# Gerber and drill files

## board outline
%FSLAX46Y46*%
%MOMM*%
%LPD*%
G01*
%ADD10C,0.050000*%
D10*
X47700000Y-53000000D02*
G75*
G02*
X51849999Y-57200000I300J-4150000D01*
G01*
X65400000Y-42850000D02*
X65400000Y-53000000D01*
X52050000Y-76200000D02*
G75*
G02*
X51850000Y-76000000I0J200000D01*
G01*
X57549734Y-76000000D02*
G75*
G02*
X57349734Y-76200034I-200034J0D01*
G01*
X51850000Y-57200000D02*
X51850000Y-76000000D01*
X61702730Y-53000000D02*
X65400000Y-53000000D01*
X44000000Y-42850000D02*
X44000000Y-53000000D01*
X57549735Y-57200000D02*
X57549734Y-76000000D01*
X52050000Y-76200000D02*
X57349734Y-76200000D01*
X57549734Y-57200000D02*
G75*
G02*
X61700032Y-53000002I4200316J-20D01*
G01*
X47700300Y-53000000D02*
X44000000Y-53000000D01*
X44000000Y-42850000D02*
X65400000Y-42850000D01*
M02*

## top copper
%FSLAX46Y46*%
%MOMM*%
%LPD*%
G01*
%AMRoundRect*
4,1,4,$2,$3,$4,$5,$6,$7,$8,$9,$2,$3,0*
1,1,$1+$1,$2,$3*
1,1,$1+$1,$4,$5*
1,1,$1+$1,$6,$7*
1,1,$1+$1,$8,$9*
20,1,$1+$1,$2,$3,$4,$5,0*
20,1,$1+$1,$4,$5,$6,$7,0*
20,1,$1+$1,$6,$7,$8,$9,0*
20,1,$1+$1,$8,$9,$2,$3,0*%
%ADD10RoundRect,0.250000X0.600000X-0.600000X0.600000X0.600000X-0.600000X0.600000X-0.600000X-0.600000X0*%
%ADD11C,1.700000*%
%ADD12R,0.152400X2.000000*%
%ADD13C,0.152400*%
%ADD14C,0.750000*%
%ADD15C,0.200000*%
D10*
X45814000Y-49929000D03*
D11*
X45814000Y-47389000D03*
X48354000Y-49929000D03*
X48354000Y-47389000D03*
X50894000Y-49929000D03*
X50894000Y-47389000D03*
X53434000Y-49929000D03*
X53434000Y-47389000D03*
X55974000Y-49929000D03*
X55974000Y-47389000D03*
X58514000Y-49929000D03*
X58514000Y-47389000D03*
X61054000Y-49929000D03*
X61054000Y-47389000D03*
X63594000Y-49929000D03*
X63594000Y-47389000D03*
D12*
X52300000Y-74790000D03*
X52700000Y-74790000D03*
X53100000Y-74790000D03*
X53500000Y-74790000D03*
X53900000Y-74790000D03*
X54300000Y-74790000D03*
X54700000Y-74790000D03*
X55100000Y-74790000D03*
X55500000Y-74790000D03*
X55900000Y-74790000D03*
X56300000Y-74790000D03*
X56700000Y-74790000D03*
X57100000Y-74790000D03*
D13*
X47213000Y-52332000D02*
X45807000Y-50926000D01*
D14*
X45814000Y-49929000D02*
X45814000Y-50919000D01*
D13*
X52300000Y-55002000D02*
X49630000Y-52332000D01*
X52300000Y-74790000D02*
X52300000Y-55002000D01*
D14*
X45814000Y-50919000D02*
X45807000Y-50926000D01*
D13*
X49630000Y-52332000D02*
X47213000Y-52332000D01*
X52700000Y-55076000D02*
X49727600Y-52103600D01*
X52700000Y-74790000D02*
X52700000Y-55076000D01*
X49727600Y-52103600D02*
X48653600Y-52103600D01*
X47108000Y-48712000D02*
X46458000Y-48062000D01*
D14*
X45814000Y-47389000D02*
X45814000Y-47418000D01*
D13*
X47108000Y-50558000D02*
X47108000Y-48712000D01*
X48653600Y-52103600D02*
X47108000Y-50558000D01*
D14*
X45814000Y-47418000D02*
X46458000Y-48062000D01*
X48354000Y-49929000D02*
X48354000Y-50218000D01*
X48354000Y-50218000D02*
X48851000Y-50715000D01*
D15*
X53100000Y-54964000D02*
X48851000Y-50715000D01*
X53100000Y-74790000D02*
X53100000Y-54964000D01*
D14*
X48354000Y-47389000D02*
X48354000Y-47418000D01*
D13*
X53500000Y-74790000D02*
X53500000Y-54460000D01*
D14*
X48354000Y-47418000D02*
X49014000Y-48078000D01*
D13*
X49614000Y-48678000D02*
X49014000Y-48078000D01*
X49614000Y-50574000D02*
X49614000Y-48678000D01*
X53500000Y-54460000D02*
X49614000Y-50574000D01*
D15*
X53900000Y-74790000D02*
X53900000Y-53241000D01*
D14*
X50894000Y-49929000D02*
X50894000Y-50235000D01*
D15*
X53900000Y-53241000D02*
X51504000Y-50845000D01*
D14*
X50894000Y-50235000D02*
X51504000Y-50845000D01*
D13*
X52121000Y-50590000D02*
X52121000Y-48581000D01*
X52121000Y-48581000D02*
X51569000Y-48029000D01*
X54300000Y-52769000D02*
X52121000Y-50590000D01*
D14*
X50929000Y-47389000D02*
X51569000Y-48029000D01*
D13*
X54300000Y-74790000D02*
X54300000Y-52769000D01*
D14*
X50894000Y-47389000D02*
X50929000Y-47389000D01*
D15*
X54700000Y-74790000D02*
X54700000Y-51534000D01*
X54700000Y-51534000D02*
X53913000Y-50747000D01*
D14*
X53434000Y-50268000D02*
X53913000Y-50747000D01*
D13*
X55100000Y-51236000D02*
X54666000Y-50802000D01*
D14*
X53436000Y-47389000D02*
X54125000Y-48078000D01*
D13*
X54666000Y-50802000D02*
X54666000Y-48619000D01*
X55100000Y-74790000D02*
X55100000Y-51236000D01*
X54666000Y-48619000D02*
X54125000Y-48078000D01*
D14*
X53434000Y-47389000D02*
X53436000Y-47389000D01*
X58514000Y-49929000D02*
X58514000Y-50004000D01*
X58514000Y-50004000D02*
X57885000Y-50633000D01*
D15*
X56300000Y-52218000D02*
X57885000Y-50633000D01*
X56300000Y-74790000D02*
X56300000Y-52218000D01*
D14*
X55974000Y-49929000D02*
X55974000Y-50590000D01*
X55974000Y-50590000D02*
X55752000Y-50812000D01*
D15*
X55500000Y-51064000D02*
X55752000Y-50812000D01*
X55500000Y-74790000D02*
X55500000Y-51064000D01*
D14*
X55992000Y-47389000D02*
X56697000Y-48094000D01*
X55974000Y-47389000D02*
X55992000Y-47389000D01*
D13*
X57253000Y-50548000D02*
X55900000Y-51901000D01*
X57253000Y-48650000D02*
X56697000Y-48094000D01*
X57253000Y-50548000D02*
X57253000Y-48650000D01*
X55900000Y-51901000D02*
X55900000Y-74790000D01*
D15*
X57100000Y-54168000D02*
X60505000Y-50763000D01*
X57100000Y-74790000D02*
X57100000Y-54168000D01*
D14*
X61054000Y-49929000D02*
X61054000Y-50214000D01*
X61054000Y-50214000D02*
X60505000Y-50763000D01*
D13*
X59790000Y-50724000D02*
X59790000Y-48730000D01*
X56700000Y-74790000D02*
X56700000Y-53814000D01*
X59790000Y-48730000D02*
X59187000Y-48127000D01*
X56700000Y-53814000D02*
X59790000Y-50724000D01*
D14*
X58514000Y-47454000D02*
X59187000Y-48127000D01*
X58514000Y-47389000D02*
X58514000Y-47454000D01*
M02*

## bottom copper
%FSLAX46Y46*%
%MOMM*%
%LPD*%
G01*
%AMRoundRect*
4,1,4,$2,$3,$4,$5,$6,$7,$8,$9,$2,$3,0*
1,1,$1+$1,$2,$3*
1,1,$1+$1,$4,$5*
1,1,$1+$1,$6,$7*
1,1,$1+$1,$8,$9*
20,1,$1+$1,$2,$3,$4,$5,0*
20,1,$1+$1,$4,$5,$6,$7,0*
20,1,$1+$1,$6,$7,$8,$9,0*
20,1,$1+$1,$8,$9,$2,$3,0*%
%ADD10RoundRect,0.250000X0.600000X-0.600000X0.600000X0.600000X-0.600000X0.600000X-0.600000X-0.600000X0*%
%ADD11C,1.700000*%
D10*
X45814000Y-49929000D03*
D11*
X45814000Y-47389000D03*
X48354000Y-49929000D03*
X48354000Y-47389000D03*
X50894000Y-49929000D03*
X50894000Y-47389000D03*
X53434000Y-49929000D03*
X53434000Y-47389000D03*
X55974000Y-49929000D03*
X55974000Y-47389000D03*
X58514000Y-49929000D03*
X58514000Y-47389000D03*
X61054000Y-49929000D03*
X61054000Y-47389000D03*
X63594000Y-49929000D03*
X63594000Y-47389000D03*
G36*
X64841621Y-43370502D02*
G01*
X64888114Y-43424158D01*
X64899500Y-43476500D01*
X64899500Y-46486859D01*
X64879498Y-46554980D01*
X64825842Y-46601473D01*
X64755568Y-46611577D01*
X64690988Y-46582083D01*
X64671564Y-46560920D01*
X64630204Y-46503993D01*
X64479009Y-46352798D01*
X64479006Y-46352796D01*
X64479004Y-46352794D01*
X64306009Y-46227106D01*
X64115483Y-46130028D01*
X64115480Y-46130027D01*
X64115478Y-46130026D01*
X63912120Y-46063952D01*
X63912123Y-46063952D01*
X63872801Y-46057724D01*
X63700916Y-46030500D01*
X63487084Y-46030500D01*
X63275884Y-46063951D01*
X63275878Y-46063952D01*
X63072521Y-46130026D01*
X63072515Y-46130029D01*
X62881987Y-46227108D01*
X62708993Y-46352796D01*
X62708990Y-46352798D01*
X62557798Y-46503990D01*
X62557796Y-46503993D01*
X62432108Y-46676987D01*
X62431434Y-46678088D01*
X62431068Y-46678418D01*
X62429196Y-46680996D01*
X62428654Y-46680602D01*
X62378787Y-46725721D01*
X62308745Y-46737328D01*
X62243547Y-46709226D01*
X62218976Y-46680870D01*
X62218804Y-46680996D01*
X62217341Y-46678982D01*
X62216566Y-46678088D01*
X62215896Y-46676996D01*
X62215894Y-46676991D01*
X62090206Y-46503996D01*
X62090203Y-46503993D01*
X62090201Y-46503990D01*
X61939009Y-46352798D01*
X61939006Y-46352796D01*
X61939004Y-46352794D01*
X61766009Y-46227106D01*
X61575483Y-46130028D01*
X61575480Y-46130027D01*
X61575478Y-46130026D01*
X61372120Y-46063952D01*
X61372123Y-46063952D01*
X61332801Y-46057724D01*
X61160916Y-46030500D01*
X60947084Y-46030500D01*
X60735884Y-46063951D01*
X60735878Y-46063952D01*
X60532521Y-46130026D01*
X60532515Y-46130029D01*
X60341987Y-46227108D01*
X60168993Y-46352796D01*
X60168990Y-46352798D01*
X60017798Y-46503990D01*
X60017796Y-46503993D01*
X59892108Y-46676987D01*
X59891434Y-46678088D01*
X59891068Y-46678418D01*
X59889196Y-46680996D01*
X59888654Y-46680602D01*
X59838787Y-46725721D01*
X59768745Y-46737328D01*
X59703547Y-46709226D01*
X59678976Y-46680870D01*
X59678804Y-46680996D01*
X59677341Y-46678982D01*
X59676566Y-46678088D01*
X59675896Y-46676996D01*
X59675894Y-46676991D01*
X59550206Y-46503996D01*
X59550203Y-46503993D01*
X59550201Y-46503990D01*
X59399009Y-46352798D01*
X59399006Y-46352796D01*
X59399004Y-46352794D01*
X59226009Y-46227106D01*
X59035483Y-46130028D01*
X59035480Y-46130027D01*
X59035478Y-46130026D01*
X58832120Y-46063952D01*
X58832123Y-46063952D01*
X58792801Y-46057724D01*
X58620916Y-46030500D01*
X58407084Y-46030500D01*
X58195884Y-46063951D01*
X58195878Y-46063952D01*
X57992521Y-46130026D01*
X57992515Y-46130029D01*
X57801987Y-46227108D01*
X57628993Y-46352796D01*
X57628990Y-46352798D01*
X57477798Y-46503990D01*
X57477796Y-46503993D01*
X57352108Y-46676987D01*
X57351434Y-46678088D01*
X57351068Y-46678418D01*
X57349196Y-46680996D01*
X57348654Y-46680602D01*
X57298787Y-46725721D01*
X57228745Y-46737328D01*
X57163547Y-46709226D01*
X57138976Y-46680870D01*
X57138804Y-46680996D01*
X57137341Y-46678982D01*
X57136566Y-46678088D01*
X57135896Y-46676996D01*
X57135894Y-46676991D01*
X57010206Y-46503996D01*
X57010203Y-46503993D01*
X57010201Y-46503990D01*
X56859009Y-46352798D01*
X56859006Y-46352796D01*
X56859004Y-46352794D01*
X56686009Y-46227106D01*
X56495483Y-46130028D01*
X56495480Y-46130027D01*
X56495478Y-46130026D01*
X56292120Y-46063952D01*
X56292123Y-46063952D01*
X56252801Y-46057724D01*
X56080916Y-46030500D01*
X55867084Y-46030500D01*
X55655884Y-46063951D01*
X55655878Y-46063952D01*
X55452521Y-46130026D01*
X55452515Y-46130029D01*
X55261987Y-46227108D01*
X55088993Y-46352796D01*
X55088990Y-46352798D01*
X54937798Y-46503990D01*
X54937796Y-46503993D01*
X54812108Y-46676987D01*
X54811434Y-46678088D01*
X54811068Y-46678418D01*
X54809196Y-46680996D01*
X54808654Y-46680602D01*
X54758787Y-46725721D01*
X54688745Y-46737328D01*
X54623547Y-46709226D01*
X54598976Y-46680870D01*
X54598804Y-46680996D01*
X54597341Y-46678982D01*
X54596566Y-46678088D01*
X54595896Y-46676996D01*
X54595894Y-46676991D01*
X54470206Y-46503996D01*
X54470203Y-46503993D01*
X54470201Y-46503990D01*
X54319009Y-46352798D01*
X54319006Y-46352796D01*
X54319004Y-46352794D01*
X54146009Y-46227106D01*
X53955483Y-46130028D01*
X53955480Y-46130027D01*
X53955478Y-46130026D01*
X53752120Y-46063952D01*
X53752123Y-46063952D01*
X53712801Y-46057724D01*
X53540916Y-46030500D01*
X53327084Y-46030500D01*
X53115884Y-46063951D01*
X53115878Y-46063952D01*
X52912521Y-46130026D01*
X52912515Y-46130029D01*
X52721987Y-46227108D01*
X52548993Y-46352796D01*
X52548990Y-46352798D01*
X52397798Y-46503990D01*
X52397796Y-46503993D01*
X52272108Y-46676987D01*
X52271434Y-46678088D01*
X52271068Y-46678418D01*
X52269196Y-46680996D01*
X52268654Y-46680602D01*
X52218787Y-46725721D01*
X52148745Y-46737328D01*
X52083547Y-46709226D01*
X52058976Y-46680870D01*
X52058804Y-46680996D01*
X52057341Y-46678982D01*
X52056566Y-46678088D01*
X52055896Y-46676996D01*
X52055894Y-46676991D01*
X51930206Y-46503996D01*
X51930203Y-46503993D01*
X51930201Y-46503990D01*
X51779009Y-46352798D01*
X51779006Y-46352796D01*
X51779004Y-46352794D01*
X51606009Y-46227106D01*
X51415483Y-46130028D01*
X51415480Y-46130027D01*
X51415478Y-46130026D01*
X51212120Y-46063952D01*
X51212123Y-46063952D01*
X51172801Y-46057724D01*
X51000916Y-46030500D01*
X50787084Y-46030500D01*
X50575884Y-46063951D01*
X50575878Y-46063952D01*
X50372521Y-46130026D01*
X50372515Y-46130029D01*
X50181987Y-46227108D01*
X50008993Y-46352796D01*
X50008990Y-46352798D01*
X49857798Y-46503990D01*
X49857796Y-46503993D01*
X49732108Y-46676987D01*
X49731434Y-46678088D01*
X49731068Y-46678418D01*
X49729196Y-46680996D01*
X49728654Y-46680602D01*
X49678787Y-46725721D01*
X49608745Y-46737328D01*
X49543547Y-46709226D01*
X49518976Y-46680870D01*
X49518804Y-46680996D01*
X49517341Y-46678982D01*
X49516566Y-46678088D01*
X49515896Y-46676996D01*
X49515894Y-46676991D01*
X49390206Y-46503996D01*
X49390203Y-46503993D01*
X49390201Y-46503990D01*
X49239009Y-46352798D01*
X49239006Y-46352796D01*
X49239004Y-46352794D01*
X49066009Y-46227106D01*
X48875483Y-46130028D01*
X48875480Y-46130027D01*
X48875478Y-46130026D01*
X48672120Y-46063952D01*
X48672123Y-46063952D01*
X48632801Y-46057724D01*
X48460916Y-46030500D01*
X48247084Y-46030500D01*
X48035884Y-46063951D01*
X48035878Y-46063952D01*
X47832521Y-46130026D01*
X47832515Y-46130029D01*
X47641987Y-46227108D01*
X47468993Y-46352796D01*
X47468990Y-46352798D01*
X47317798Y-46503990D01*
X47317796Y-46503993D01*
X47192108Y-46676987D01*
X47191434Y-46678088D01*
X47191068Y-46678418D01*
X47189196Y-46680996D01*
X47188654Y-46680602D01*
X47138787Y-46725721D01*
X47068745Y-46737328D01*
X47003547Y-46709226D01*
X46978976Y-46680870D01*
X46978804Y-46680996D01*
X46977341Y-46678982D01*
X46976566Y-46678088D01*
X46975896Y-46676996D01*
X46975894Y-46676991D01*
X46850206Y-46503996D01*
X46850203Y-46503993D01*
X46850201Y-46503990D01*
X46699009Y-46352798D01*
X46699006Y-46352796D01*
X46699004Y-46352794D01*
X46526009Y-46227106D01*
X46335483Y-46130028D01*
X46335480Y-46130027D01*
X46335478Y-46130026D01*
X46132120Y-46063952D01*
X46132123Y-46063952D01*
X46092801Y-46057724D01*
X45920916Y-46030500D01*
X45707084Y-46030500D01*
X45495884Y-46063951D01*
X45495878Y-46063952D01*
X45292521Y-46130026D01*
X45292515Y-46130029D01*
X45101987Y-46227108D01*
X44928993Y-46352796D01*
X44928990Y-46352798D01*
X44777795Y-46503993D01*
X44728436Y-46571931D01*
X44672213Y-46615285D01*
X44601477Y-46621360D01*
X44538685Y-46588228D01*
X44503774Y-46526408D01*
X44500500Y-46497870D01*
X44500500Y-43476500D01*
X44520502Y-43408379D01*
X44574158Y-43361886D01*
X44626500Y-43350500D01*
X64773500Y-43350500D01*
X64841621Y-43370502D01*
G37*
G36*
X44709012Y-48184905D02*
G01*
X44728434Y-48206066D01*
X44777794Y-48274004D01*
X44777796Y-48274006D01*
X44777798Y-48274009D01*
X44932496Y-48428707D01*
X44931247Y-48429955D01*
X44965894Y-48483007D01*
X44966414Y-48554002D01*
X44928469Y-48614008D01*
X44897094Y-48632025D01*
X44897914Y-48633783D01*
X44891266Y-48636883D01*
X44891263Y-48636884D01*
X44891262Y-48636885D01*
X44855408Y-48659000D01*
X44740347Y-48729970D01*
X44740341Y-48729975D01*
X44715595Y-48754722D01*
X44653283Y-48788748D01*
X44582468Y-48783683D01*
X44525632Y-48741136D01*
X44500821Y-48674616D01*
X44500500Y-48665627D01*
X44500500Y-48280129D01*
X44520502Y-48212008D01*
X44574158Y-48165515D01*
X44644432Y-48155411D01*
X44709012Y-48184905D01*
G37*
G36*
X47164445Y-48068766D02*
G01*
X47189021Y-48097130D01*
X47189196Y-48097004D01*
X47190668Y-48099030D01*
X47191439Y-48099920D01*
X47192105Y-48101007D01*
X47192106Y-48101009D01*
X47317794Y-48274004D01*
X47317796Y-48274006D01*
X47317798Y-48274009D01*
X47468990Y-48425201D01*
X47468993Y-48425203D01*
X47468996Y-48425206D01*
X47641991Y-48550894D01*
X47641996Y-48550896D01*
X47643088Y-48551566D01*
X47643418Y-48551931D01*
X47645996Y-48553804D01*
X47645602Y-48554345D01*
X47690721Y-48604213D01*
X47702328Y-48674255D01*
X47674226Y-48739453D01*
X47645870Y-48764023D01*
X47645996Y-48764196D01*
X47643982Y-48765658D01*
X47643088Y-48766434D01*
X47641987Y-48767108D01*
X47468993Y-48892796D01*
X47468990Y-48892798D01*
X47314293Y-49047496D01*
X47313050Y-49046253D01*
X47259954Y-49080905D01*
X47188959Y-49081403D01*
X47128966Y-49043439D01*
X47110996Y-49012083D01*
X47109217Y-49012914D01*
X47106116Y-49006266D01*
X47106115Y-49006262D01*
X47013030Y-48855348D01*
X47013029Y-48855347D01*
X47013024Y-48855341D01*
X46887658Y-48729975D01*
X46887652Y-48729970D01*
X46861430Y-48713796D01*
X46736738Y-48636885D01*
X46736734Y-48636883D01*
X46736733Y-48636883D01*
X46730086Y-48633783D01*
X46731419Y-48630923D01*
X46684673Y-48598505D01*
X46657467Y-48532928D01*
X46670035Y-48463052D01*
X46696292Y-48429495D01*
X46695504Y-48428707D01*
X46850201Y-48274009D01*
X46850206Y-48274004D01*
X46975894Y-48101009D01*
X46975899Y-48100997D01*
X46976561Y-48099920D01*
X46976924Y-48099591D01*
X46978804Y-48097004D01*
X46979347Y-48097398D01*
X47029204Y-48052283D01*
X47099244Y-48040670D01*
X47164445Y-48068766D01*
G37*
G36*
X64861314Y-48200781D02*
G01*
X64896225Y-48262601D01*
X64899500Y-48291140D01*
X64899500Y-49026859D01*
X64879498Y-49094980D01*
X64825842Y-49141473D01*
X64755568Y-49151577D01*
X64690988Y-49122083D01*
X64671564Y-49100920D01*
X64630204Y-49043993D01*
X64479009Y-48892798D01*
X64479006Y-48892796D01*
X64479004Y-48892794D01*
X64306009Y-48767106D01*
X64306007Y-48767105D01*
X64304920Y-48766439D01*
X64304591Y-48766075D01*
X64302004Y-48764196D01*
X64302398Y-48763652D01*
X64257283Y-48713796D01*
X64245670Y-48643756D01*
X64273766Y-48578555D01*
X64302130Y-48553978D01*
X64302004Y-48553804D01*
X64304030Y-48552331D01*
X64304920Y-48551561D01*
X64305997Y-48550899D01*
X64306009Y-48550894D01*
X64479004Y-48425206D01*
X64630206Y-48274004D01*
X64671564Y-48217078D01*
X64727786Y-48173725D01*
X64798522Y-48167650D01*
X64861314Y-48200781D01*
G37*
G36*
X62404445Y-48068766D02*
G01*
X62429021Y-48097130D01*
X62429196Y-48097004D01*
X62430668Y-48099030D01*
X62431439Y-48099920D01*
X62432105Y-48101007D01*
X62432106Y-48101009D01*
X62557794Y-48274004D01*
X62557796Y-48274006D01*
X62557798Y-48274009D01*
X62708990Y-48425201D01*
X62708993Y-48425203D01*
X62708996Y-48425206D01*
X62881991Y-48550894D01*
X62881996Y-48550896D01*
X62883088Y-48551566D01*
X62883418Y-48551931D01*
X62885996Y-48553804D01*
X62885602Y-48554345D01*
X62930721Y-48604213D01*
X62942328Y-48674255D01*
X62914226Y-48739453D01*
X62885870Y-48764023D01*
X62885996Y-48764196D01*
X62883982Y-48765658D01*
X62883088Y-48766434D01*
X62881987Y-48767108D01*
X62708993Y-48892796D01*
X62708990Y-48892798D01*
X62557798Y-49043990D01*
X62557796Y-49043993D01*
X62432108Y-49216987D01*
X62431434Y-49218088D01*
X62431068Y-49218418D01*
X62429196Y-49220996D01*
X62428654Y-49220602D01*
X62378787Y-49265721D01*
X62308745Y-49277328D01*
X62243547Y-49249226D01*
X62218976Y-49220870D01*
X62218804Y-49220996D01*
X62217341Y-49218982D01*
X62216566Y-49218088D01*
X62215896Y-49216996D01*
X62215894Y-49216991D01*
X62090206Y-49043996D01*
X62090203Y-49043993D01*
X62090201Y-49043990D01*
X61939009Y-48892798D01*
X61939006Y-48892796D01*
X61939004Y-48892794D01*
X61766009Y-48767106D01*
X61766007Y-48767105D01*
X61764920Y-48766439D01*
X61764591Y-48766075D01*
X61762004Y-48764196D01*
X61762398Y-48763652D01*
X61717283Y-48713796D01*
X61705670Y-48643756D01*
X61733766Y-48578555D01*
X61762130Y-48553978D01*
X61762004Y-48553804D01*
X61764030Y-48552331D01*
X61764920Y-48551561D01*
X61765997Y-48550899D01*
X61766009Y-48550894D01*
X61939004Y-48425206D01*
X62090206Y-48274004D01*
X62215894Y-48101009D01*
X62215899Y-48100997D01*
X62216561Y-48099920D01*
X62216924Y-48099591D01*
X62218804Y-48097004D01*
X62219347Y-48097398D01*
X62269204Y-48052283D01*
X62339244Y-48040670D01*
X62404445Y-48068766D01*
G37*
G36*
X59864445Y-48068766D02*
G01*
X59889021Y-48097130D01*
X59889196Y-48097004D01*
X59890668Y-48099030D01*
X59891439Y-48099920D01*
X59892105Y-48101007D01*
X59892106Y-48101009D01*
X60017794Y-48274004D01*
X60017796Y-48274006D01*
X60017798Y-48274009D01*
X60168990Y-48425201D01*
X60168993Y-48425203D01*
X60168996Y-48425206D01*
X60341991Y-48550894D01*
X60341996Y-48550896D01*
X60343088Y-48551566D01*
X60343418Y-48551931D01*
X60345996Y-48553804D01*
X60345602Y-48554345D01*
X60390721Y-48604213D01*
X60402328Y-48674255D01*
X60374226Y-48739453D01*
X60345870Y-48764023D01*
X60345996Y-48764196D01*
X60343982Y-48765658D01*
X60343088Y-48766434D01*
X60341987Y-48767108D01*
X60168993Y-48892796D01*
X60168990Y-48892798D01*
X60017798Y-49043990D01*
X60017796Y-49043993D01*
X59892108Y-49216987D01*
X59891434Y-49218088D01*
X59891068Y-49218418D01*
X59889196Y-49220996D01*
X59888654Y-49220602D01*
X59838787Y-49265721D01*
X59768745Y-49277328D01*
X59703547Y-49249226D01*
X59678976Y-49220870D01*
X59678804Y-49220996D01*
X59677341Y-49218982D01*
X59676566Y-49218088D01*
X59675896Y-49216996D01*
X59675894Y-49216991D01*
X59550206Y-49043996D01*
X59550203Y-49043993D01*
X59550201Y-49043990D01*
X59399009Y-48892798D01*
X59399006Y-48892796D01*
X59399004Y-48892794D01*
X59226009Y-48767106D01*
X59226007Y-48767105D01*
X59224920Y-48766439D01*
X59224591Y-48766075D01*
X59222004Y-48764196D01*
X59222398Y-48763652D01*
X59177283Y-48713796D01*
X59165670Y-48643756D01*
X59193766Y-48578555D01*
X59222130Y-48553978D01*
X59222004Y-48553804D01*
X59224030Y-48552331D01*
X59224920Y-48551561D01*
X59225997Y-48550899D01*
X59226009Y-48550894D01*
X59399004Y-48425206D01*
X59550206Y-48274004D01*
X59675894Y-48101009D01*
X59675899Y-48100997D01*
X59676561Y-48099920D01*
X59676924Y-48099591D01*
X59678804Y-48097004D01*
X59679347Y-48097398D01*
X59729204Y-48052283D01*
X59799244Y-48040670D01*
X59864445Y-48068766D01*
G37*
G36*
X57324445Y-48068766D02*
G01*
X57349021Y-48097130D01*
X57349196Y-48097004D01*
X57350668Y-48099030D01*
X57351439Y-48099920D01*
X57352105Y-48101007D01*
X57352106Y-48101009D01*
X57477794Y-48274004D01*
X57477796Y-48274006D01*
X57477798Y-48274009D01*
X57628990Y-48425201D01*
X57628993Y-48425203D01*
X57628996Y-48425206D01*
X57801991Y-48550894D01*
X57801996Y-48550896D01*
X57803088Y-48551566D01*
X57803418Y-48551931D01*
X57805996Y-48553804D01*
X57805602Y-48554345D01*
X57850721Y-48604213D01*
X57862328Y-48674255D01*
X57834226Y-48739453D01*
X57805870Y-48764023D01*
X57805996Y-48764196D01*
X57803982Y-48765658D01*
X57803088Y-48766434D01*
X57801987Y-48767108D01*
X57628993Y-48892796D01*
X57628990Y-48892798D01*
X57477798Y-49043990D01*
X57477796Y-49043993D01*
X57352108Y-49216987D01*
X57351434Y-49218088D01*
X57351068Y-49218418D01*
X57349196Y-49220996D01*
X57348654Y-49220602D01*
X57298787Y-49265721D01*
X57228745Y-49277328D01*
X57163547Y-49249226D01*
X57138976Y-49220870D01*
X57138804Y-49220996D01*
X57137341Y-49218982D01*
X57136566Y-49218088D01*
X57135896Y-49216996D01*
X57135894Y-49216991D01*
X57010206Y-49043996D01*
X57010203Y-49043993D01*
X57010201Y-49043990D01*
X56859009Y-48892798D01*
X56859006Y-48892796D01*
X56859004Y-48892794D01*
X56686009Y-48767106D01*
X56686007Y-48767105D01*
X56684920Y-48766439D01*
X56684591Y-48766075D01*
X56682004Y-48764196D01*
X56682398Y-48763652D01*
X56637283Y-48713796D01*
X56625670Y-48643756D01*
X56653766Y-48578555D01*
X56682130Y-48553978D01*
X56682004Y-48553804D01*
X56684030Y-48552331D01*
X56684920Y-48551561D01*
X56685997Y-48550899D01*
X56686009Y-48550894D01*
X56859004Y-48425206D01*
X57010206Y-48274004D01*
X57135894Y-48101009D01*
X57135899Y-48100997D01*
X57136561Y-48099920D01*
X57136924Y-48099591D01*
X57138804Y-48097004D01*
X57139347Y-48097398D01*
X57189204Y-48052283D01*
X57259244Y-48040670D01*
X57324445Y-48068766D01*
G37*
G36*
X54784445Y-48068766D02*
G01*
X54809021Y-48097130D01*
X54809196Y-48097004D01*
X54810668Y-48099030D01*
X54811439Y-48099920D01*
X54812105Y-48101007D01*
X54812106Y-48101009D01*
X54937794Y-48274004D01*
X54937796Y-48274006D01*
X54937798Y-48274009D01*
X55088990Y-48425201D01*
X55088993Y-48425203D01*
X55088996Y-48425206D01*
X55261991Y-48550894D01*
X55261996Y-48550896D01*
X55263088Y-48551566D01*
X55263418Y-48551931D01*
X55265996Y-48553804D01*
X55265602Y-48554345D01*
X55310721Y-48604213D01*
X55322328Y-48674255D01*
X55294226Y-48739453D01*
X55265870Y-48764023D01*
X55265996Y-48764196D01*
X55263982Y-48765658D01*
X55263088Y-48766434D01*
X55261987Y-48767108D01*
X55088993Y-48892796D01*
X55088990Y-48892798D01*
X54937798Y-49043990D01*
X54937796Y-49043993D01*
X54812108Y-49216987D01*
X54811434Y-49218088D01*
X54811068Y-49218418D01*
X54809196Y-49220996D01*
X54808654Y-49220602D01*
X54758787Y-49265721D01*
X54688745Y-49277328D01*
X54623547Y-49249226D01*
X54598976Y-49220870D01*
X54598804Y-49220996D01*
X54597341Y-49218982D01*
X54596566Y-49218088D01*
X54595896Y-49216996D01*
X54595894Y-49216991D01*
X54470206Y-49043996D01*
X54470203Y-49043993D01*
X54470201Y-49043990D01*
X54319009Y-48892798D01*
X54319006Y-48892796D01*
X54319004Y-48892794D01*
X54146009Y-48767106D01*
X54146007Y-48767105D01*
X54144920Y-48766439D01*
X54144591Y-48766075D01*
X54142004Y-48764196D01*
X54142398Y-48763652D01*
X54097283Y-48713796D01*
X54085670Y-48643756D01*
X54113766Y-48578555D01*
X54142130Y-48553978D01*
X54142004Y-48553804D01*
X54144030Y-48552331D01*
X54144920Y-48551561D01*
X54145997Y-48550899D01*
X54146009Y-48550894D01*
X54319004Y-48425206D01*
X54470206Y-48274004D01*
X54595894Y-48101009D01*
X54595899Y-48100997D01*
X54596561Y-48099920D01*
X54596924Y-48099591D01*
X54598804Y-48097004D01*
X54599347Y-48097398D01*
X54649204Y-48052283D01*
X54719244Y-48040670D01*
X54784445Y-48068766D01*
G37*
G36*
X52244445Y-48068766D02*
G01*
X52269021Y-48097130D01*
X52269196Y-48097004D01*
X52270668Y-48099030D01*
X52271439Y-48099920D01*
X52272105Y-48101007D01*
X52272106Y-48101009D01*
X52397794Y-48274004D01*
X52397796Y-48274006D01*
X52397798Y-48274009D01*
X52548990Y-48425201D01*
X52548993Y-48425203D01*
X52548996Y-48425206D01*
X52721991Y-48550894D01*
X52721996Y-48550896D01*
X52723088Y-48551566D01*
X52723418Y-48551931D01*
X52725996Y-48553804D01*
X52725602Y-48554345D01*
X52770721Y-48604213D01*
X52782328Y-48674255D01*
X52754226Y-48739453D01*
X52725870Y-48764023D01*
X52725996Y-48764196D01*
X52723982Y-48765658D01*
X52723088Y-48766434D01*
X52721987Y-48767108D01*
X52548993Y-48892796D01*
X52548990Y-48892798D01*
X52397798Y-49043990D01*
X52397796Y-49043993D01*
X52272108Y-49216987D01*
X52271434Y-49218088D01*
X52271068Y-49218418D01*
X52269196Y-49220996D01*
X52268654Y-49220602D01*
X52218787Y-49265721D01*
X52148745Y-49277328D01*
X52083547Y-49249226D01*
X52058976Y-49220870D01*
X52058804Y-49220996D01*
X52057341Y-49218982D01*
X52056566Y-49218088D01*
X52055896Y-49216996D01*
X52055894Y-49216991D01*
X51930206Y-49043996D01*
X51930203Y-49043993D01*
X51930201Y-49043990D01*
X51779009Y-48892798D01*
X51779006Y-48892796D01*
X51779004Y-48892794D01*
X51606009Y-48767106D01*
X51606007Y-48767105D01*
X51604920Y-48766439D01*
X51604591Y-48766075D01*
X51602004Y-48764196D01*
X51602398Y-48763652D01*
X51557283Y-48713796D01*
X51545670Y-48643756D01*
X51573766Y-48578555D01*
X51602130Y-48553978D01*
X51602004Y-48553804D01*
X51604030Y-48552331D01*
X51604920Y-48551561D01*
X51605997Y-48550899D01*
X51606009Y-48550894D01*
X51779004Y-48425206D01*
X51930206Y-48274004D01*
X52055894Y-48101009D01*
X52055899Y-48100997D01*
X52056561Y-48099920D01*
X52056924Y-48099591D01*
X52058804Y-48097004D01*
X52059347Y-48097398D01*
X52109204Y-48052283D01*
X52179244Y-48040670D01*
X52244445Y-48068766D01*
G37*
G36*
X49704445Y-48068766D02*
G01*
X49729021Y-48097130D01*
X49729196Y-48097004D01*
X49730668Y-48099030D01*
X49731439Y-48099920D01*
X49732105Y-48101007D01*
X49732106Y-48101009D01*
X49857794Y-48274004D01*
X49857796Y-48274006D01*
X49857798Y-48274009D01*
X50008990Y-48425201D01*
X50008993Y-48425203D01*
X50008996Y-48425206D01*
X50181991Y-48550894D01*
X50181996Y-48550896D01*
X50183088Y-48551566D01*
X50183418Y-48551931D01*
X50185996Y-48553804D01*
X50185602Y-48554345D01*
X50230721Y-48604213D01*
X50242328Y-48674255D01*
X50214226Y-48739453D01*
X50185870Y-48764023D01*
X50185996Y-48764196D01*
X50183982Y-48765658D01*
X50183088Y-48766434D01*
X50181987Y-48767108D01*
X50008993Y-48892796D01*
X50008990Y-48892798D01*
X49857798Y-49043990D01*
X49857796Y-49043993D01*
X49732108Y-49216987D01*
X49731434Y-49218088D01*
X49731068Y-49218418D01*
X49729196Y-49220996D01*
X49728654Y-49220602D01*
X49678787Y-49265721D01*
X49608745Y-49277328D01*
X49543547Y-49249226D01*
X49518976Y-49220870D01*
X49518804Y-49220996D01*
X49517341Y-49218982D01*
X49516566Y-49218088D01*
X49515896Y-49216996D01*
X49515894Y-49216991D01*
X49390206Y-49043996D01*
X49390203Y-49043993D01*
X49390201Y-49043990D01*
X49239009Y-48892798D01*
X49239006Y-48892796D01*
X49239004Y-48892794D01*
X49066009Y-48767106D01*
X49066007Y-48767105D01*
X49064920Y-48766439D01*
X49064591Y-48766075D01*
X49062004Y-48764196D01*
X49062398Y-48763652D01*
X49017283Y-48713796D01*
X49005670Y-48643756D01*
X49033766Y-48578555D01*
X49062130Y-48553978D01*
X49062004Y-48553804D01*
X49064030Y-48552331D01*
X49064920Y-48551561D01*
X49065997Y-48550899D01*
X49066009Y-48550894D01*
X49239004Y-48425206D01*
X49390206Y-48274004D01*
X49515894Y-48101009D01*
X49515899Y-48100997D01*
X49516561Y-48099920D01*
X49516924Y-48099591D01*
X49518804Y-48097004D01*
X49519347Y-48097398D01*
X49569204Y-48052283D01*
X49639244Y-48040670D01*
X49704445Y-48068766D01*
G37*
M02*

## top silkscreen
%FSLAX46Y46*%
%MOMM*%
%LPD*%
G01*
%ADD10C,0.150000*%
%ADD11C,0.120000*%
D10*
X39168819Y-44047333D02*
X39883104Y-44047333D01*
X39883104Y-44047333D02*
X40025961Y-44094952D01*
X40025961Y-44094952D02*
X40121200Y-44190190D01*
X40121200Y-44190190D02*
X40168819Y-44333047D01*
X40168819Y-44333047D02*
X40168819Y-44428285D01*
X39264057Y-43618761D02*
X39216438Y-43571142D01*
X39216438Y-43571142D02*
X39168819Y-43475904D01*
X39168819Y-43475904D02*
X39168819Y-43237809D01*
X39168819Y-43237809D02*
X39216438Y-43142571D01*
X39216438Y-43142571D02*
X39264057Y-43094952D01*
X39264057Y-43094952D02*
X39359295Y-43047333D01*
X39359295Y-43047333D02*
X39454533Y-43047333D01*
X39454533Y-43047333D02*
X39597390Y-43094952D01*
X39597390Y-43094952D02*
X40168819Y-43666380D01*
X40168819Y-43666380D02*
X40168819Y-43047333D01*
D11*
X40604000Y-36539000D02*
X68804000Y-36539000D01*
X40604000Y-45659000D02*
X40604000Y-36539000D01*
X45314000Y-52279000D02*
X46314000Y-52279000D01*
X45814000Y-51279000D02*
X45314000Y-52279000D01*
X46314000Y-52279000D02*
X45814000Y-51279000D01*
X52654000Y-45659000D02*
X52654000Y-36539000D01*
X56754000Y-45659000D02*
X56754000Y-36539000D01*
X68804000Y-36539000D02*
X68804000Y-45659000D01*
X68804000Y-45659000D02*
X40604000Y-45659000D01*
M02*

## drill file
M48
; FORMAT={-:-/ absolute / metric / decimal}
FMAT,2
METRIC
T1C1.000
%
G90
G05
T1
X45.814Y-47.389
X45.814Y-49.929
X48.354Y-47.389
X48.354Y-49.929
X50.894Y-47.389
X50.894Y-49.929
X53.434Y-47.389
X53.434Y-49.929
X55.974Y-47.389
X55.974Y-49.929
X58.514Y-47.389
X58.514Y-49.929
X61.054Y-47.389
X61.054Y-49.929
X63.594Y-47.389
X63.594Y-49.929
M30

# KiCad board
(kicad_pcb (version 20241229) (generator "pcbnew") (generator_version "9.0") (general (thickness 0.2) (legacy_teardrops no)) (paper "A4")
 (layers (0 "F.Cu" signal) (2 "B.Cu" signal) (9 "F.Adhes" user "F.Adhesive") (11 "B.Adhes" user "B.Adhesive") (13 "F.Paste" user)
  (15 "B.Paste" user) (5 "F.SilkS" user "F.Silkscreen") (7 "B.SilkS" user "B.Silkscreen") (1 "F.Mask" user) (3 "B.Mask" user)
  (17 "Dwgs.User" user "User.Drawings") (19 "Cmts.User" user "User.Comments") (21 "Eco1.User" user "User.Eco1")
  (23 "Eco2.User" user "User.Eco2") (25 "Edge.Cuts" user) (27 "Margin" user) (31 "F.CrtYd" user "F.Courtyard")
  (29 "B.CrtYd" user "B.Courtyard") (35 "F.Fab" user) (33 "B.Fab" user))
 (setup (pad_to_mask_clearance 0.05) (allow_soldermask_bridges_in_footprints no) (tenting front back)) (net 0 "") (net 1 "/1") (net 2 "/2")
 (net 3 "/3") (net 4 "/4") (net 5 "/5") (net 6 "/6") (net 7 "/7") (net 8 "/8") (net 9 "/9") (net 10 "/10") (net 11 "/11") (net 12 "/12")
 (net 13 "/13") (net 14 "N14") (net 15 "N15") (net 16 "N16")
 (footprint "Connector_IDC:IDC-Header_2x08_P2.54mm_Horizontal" (layer "F.Cu") (at 45.814 49.929 90)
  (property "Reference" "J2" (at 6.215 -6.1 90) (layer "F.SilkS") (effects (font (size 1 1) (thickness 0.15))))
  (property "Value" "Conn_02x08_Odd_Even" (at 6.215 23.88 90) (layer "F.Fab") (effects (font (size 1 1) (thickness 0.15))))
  (fp_line (start 13.39 -5.21) (end 13.39 22.99) (stroke (width 0.12) (type solid)) (layer "F.SilkS"))
  (fp_line (start 4.27 -5.21) (end 13.39 -5.21) (stroke (width 0.12) (type solid)) (layer "F.SilkS"))
  (fp_line (start -2.35 -0.5) (end -2.35 0.5) (stroke (width 0.12) (type solid)) (layer "F.SilkS"))
  (fp_line (start -1.35 0) (end -2.35 -0.5) (stroke (width 0.12) (type solid)) (layer "F.SilkS"))
  (fp_line (start -2.35 0.5) (end -1.35 0) (stroke (width 0.12) (type solid)) (layer "F.SilkS"))
  (fp_line (start 4.27 6.84) (end 13.39 6.84) (stroke (width 0.12) (type solid)) (layer "F.SilkS"))
  (fp_line (start 4.27 10.94) (end 13.39 10.94) (stroke (width 0.12) (type solid)) (layer "F.SilkS"))
  (fp_line (start 13.39 22.99) (end 4.27 22.99) (stroke (width 0.12) (type solid)) (layer "F.SilkS"))
  (fp_line (start 4.27 22.99) (end 4.27 -5.21) (stroke (width 0.12) (type solid)) (layer "F.SilkS"))
  (pad "1" thru_hole roundrect (at 0 0 90) (size 1.7 1.7) (drill 1) (layers "*.Cu" "*.Mask") (remove_unused_layers no)
   (roundrect_rratio 0.147059) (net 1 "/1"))
  (pad "2" thru_hole circle (at 2.54 0 90) (size 1.7 1.7) (drill 1) (layers "*.Cu" "*.Mask") (remove_unused_layers no) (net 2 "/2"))
  (pad "3" thru_hole circle (at 0 2.54 90) (size 1.7 1.7) (drill 1) (layers "*.Cu" "*.Mask") (remove_unused_layers no) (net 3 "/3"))
  (pad "4" thru_hole circle (at 2.54 2.54 90) (size 1.7 1.7) (drill 1) (layers "*.Cu" "*.Mask") (remove_unused_layers no) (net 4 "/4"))
  (pad "5" thru_hole circle (at 0 5.08 90) (size 1.7 1.7) (drill 1) (layers "*.Cu" "*.Mask") (remove_unused_layers no) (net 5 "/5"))
  (pad "6" thru_hole circle (at 2.54 5.08 90) (size 1.7 1.7) (drill 1) (layers "*.Cu" "*.Mask") (remove_unused_layers no) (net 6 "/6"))
  (pad "7" thru_hole circle (at 0 7.62 90) (size 1.7 1.7) (drill 1) (layers "*.Cu" "*.Mask") (remove_unused_layers no) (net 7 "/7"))
  (pad "8" thru_hole circle (at 2.54 7.62 90) (size 1.7 1.7) (drill 1) (layers "*.Cu" "*.Mask") (remove_unused_layers no) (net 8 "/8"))
  (pad "9" thru_hole circle (at 0 10.16 90) (size 1.7 1.7) (drill 1) (layers "*.Cu" "*.Mask") (remove_unused_layers no) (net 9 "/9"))
  (pad "10" thru_hole circle (at 2.54 10.16 90) (size 1.7 1.7) (drill 1) (layers "*.Cu" "*.Mask") (remove_unused_layers no) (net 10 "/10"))
  (pad "11" thru_hole circle (at 0 12.7 90) (size 1.7 1.7) (drill 1) (layers "*.Cu" "*.Mask") (remove_unused_layers no) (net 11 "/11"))
  (pad "12" thru_hole circle (at 2.54 12.7 90) (size 1.7 1.7) (drill 1) (layers "*.Cu" "*.Mask") (remove_unused_layers no) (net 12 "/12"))
  (pad "13" thru_hole circle (at 0 15.24 90) (size 1.7 1.7) (drill 1) (layers "*.Cu" "*.Mask") (remove_unused_layers no) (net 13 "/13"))
  (pad "14" thru_hole circle (at 2.54 15.24 90) (size 1.7 1.7) (drill 1) (layers "*.Cu" "*.Mask") (remove_unused_layers no) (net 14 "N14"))
  (pad "15" thru_hole circle (at 0 17.78 90) (size 1.7 1.7) (drill 1) (layers "*.Cu" "*.Mask") (remove_unused_layers no) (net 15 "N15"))
  (pad "16" thru_hole circle (at 2.54 17.78 90) (size 1.7 1.7) (drill 1) (layers "*.Cu" "*.Mask") (remove_unused_layers no) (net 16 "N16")))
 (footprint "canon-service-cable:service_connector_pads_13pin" (layer "F.Cu") (at 52.3 75.79)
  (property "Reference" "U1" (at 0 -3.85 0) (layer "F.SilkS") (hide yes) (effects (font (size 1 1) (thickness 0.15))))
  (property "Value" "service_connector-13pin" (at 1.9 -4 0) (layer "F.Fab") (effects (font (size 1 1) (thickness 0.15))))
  (pad "1" smd rect (at 0 -1) (size 0.1524 2) (layers "F.Cu" "F.Mask" "F.Paste") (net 1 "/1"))
  (pad "2" smd rect (at 0.4 -1) (size 0.1524 2) (layers "F.Cu" "F.Mask" "F.Paste") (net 2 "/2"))
  (pad "3" smd rect (at 0.8 -1) (size 0.1524 2) (layers "F.Cu" "F.Mask" "F.Paste") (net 3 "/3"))
  (pad "4" smd rect (at 1.2 -1) (size 0.1524 2) (layers "F.Cu" "F.Mask" "F.Paste") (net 4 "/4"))
  (pad "5" smd rect (at 1.6 -1) (size 0.1524 2) (layers "F.Cu" "F.Mask" "F.Paste") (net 5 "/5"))
  (pad "6" smd rect (at 2 -1) (size 0.1524 2) (layers "F.Cu" "F.Mask" "F.Paste") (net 6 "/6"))
  (pad "7" smd rect (at 2.4 -1) (size 0.1524 2) (layers "F.Cu" "F.Mask" "F.Paste") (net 7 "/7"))
  (pad "8" smd rect (at 2.8 -1) (size 0.1524 2) (layers "F.Cu" "F.Mask" "F.Paste") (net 8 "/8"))
  (pad "9" smd rect (at 3.2 -1) (size 0.1524 2) (layers "F.Cu" "F.Mask" "F.Paste") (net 9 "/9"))
  (pad "10" smd rect (at 3.6 -1) (size 0.1524 2) (layers "F.Cu" "F.Mask" "F.Paste") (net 10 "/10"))
  (pad "11" smd rect (at 4 -1) (size 0.1524 2) (layers "F.Cu" "F.Mask" "F.Paste") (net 11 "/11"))
  (pad "12" smd rect (at 4.4 -1) (size 0.1524 2) (layers "F.Cu" "F.Mask" "F.Paste") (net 12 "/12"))
  (pad "13" smd rect (at 4.8 -1) (size 0.1524 2) (layers "F.Cu" "F.Mask" "F.Paste") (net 13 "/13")))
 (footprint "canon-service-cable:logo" (layer "B.Cu") (at 52.784938 54.543327 180)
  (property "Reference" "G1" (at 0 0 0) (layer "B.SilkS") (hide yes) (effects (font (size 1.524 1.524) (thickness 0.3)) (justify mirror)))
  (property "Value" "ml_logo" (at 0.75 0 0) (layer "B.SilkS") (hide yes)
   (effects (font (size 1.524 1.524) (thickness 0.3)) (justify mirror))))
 (gr_arc (start 47.7 53) (mid 50.652312 54.233131) (end 51.85 57.2) (stroke (width 0.05) (type solid)) (layer "Edge.Cuts"))
 (gr_line (start 65.4 42.85) (end 65.4 53) (stroke (width 0.05) (type default)) (layer "Edge.Cuts"))
 (gr_arc (start 52.05 76.2) (mid 51.908579 76.141421) (end 51.85 76) (stroke (width 0.05) (type solid)) (layer "Edge.Cuts"))
 (gr_arc (start 57.549734 76) (mid 57.491155 76.141421) (end 57.349734 76.2) (stroke (width 0.05) (type solid)) (layer "Edge.Cuts"))
 (gr_line (start 51.85 57.2) (end 51.85 76) (stroke (width 0.05) (type default)) (layer "Edge.Cuts"))
 (gr_line (start 61.70273 53) (end 65.4 53) (stroke (width 0.05) (type default)) (layer "Edge.Cuts"))
 (gr_line (start 44 42.85) (end 44 53) (stroke (width 0.05) (type default)) (layer "Edge.Cuts"))
 (gr_line (start 57.549735 57.2) (end 57.549734 76) (stroke (width 0.05) (type default)) (layer "Edge.Cuts"))
 (gr_line (start 52.05 76.2) (end 57.349734 76.2) (stroke (width 0.05) (type default)) (layer "Edge.Cuts"))
 (gr_arc (start 57.549734 57.2) (mid 58.762349 54.247683) (end 61.700032 53) (stroke (width 0.05) (type solid)) (layer "Edge.Cuts"))
 (gr_line (start 47.7003 53) (end 44 53) (stroke (width 0.05) (type default)) (layer "Edge.Cuts"))
 (gr_line (start 44 42.85) (end 65.4 42.85) (stroke (width 0.05) (type solid)) (layer "Edge.Cuts"))
 (segment (start 47.213 52.332) (end 45.807 50.926) (width 0.1524) (layer "F.Cu") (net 1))
 (segment (start 45.814 49.929) (end 45.814 50.919) (width 0.75) (layer "F.Cu") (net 1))
 (segment (start 52.3 55.002) (end 49.63 52.332) (width 0.1524) (layer "F.Cu") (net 1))
 (segment (start 52.3 74.79) (end 52.3 55.002) (width 0.1524) (layer "F.Cu") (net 1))
 (segment (start 45.814 50.919) (end 45.807 50.926) (width 0.75) (layer "F.Cu") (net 1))
 (segment (start 49.63 52.332) (end 47.213 52.332) (width 0.1524) (layer "F.Cu") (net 1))
 (segment (start 52.7 55.076) (end 49.7276 52.1036) (width 0.1524) (layer "F.Cu") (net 2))
 (segment (start 52.7 74.79) (end 52.7 55.076) (width 0.1524) (layer "F.Cu") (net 2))
 (segment (start 49.7276 52.1036) (end 48.6536 52.1036) (width 0.1524) (layer "F.Cu") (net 2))
 (segment (start 47.108 48.712) (end 46.458 48.062) (width 0.1524) (layer "F.Cu") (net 2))
 (segment (start 45.814 47.389) (end 45.814 47.418) (width 0.75) (layer "F.Cu") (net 2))
 (segment (start 47.108 50.558) (end 47.108 48.712) (width 0.1524) (layer "F.Cu") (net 2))
 (segment (start 48.6536 52.1036) (end 47.108 50.558) (width 0.1524) (layer "F.Cu") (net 2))
 (segment (start 45.814 47.418) (end 46.458 48.062) (width 0.75) (layer "F.Cu") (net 2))
 (segment (start 48.354 49.929) (end 48.354 50.218) (width 0.75) (layer "F.Cu") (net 3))
 (segment (start 48.354 50.218) (end 48.851 50.715) (width 0.75) (layer "F.Cu") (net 3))
 (segment (start 53.1 54.964) (end 48.851 50.715) (width 0.2) (layer "F.Cu") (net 3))
 (segment (start 53.1 74.79) (end 53.1 54.964) (width 0.2) (layer "F.Cu") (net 3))
 (segment (start 48.354 47.389) (end 48.354 47.418) (width 0.75) (layer "F.Cu") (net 4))
 (segment (start 53.5 74.79) (end 53.5 54.46) (width 0.1524) (layer "F.Cu") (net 4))
 (segment (start 48.354 47.418) (end 49.014 48.078) (width 0.75) (layer "F.Cu") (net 4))
 (segment (start 49.614 48.678) (end 49.014 48.078) (width 0.1524) (layer "F.Cu") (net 4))
 (segment (start 49.614 50.574) (end 49.614 48.678) (width 0.1524) (layer "F.Cu") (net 4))
 (segment (start 53.5 54.46) (end 49.614 50.574) (width 0.1524) (layer "F.Cu") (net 4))
 (segment (start 53.9 74.79) (end 53.9 53.241) (width 0.2) (layer "F.Cu") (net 5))
 (segment (start 50.894 49.929) (end 50.894 50.235) (width 0.75) (layer "F.Cu") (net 5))
 (segment (start 53.9 53.241) (end 51.504 50.845) (width 0.2) (layer "F.Cu") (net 5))
 (segment (start 50.894 50.235) (end 51.504 50.845) (width 0.75) (layer "F.Cu") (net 5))
 (segment (start 52.121 50.59) (end 52.121 48.581) (width 0.1524) (layer "F.Cu") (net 6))
 (segment (start 52.121 48.581) (end 51.569 48.029) (width 0.1524) (layer "F.Cu") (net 6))
 (segment (start 54.3 52.769) (end 52.121 50.59) (width 0.1524) (layer "F.Cu") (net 6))
 (segment (start 50.929 47.389) (end 51.569 48.029) (width 0.75) (layer "F.Cu") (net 6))
 (segment (start 54.3 74.79) (end 54.3 52.769) (width 0.1524) (layer "F.Cu") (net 6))
 (segment (start 50.894 47.389) (end 50.929 47.389) (width 0.75) (layer "F.Cu") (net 6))
 (segment (start 54.7 74.79) (end 54.7 51.534) (width 0.2) (layer "F.Cu") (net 7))
 (segment (start 54.7 51.534) (end 53.913 50.747) (width 0.2) (layer "F.Cu") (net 7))
 (segment (start 53.434 50.268) (end 53.913 50.747) (width 0.75) (layer "F.Cu") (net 7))
 (segment (start 55.1 51.236) (end 54.666 50.802) (width 0.1524) (layer "F.Cu") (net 8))
 (segment (start 53.436 47.389) (end 54.125 48.078) (width 0.75) (layer "F.Cu") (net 8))
 (segment (start 54.666 50.802) (end 54.666 48.619) (width 0.1524) (layer "F.Cu") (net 8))
 (segment (start 55.1 74.79) (end 55.1 51.236) (width 0.1524) (layer "F.Cu") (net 8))
 (segment (start 54.666 48.619) (end 54.125 48.078) (width 0.1524) (layer "F.Cu") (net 8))
 (segment (start 53.434 47.389) (end 53.436 47.389) (width 0.75) (layer "F.Cu") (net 8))
 (segment (start 58.514 49.929) (end 58.514 50.004) (width 0.75) (layer "F.Cu") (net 11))
 (segment (start 58.514 50.004) (end 57.885 50.633) (width 0.75) (layer "F.Cu") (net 11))
 (segment (start 56.3 52.218) (end 57.885 50.633) (width 0.2) (layer "F.Cu") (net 11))
 (segment (start 56.3 74.79) (end 56.3 52.218) (width 0.2) (layer "F.Cu") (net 11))
 (segment (start 55.974 49.929) (end 55.974 50.59) (width 0.75) (layer "F.Cu") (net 9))
 (segment (start 55.974 50.59) (end 55.752 50.812) (width 0.75) (layer "F.Cu") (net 9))
 (segment (start 55.5 51.064) (end 55.752 50.812) (width 0.2) (layer "F.Cu") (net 9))
 (segment (start 55.5 74.79) (end 55.5 51.064) (width 0.2) (layer "F.Cu") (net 9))
 (segment (start 55.992 47.389) (end 56.697 48.094) (width 0.75) (layer "F.Cu") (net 10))
 (segment (start 55.974 47.389) (end 55.992 47.389) (width 0.75) (layer "F.Cu") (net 10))
 (segment (start 57.253 50.548) (end 55.9 51.901) (width 0.1524) (layer "F.Cu") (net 10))
 (segment (start 57.253 48.65) (end 56.697 48.094) (width 0.1524) (layer "F.Cu") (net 10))
 (segment (start 57.253 50.548) (end 57.253 48.65) (width 0.1524) (layer "F.Cu") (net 10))
 (segment (start 55.9 51.901) (end 55.9 74.79) (width 0.1524) (layer "F.Cu") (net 10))
 (segment (start 57.1 54.168) (end 60.505 50.763) (width 0.2) (layer "F.Cu") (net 13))
 (segment (start 57.1 74.79) (end 57.1 54.168) (width 0.2) (layer "F.Cu") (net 13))
 (segment (start 61.054 49.929) (end 61.054 50.214) (width 0.75) (layer "F.Cu") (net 13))
 (segment (start 61.054 50.214) (end 60.505 50.763) (width 0.75) (layer "F.Cu") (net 13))
 (segment (start 59.79 50.724) (end 59.79 48.73) (width 0.1524) (layer "F.Cu") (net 12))
 (segment (start 56.7 74.79) (end 56.7 53.814) (width 0.1524) (layer "F.Cu") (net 12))
 (segment (start 59.79 48.73) (end 59.187 48.127) (width 0.1524) (layer "F.Cu") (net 12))
 (segment (start 56.7 53.814) (end 59.79 50.724) (width 0.1524) (layer "F.Cu") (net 12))
 (segment (start 58.514 47.454) (end 59.187 48.127) (width 0.75) (layer "F.Cu") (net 12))
 (segment (start 58.514 47.389) (end 58.514 47.454) (width 0.75) (layer "F.Cu") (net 12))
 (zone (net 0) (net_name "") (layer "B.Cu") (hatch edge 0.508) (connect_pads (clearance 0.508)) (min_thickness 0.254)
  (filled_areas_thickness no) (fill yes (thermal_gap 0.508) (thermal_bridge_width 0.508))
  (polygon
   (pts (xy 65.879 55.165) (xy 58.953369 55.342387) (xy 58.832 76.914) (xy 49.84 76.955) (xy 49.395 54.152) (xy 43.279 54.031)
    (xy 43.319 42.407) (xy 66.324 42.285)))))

